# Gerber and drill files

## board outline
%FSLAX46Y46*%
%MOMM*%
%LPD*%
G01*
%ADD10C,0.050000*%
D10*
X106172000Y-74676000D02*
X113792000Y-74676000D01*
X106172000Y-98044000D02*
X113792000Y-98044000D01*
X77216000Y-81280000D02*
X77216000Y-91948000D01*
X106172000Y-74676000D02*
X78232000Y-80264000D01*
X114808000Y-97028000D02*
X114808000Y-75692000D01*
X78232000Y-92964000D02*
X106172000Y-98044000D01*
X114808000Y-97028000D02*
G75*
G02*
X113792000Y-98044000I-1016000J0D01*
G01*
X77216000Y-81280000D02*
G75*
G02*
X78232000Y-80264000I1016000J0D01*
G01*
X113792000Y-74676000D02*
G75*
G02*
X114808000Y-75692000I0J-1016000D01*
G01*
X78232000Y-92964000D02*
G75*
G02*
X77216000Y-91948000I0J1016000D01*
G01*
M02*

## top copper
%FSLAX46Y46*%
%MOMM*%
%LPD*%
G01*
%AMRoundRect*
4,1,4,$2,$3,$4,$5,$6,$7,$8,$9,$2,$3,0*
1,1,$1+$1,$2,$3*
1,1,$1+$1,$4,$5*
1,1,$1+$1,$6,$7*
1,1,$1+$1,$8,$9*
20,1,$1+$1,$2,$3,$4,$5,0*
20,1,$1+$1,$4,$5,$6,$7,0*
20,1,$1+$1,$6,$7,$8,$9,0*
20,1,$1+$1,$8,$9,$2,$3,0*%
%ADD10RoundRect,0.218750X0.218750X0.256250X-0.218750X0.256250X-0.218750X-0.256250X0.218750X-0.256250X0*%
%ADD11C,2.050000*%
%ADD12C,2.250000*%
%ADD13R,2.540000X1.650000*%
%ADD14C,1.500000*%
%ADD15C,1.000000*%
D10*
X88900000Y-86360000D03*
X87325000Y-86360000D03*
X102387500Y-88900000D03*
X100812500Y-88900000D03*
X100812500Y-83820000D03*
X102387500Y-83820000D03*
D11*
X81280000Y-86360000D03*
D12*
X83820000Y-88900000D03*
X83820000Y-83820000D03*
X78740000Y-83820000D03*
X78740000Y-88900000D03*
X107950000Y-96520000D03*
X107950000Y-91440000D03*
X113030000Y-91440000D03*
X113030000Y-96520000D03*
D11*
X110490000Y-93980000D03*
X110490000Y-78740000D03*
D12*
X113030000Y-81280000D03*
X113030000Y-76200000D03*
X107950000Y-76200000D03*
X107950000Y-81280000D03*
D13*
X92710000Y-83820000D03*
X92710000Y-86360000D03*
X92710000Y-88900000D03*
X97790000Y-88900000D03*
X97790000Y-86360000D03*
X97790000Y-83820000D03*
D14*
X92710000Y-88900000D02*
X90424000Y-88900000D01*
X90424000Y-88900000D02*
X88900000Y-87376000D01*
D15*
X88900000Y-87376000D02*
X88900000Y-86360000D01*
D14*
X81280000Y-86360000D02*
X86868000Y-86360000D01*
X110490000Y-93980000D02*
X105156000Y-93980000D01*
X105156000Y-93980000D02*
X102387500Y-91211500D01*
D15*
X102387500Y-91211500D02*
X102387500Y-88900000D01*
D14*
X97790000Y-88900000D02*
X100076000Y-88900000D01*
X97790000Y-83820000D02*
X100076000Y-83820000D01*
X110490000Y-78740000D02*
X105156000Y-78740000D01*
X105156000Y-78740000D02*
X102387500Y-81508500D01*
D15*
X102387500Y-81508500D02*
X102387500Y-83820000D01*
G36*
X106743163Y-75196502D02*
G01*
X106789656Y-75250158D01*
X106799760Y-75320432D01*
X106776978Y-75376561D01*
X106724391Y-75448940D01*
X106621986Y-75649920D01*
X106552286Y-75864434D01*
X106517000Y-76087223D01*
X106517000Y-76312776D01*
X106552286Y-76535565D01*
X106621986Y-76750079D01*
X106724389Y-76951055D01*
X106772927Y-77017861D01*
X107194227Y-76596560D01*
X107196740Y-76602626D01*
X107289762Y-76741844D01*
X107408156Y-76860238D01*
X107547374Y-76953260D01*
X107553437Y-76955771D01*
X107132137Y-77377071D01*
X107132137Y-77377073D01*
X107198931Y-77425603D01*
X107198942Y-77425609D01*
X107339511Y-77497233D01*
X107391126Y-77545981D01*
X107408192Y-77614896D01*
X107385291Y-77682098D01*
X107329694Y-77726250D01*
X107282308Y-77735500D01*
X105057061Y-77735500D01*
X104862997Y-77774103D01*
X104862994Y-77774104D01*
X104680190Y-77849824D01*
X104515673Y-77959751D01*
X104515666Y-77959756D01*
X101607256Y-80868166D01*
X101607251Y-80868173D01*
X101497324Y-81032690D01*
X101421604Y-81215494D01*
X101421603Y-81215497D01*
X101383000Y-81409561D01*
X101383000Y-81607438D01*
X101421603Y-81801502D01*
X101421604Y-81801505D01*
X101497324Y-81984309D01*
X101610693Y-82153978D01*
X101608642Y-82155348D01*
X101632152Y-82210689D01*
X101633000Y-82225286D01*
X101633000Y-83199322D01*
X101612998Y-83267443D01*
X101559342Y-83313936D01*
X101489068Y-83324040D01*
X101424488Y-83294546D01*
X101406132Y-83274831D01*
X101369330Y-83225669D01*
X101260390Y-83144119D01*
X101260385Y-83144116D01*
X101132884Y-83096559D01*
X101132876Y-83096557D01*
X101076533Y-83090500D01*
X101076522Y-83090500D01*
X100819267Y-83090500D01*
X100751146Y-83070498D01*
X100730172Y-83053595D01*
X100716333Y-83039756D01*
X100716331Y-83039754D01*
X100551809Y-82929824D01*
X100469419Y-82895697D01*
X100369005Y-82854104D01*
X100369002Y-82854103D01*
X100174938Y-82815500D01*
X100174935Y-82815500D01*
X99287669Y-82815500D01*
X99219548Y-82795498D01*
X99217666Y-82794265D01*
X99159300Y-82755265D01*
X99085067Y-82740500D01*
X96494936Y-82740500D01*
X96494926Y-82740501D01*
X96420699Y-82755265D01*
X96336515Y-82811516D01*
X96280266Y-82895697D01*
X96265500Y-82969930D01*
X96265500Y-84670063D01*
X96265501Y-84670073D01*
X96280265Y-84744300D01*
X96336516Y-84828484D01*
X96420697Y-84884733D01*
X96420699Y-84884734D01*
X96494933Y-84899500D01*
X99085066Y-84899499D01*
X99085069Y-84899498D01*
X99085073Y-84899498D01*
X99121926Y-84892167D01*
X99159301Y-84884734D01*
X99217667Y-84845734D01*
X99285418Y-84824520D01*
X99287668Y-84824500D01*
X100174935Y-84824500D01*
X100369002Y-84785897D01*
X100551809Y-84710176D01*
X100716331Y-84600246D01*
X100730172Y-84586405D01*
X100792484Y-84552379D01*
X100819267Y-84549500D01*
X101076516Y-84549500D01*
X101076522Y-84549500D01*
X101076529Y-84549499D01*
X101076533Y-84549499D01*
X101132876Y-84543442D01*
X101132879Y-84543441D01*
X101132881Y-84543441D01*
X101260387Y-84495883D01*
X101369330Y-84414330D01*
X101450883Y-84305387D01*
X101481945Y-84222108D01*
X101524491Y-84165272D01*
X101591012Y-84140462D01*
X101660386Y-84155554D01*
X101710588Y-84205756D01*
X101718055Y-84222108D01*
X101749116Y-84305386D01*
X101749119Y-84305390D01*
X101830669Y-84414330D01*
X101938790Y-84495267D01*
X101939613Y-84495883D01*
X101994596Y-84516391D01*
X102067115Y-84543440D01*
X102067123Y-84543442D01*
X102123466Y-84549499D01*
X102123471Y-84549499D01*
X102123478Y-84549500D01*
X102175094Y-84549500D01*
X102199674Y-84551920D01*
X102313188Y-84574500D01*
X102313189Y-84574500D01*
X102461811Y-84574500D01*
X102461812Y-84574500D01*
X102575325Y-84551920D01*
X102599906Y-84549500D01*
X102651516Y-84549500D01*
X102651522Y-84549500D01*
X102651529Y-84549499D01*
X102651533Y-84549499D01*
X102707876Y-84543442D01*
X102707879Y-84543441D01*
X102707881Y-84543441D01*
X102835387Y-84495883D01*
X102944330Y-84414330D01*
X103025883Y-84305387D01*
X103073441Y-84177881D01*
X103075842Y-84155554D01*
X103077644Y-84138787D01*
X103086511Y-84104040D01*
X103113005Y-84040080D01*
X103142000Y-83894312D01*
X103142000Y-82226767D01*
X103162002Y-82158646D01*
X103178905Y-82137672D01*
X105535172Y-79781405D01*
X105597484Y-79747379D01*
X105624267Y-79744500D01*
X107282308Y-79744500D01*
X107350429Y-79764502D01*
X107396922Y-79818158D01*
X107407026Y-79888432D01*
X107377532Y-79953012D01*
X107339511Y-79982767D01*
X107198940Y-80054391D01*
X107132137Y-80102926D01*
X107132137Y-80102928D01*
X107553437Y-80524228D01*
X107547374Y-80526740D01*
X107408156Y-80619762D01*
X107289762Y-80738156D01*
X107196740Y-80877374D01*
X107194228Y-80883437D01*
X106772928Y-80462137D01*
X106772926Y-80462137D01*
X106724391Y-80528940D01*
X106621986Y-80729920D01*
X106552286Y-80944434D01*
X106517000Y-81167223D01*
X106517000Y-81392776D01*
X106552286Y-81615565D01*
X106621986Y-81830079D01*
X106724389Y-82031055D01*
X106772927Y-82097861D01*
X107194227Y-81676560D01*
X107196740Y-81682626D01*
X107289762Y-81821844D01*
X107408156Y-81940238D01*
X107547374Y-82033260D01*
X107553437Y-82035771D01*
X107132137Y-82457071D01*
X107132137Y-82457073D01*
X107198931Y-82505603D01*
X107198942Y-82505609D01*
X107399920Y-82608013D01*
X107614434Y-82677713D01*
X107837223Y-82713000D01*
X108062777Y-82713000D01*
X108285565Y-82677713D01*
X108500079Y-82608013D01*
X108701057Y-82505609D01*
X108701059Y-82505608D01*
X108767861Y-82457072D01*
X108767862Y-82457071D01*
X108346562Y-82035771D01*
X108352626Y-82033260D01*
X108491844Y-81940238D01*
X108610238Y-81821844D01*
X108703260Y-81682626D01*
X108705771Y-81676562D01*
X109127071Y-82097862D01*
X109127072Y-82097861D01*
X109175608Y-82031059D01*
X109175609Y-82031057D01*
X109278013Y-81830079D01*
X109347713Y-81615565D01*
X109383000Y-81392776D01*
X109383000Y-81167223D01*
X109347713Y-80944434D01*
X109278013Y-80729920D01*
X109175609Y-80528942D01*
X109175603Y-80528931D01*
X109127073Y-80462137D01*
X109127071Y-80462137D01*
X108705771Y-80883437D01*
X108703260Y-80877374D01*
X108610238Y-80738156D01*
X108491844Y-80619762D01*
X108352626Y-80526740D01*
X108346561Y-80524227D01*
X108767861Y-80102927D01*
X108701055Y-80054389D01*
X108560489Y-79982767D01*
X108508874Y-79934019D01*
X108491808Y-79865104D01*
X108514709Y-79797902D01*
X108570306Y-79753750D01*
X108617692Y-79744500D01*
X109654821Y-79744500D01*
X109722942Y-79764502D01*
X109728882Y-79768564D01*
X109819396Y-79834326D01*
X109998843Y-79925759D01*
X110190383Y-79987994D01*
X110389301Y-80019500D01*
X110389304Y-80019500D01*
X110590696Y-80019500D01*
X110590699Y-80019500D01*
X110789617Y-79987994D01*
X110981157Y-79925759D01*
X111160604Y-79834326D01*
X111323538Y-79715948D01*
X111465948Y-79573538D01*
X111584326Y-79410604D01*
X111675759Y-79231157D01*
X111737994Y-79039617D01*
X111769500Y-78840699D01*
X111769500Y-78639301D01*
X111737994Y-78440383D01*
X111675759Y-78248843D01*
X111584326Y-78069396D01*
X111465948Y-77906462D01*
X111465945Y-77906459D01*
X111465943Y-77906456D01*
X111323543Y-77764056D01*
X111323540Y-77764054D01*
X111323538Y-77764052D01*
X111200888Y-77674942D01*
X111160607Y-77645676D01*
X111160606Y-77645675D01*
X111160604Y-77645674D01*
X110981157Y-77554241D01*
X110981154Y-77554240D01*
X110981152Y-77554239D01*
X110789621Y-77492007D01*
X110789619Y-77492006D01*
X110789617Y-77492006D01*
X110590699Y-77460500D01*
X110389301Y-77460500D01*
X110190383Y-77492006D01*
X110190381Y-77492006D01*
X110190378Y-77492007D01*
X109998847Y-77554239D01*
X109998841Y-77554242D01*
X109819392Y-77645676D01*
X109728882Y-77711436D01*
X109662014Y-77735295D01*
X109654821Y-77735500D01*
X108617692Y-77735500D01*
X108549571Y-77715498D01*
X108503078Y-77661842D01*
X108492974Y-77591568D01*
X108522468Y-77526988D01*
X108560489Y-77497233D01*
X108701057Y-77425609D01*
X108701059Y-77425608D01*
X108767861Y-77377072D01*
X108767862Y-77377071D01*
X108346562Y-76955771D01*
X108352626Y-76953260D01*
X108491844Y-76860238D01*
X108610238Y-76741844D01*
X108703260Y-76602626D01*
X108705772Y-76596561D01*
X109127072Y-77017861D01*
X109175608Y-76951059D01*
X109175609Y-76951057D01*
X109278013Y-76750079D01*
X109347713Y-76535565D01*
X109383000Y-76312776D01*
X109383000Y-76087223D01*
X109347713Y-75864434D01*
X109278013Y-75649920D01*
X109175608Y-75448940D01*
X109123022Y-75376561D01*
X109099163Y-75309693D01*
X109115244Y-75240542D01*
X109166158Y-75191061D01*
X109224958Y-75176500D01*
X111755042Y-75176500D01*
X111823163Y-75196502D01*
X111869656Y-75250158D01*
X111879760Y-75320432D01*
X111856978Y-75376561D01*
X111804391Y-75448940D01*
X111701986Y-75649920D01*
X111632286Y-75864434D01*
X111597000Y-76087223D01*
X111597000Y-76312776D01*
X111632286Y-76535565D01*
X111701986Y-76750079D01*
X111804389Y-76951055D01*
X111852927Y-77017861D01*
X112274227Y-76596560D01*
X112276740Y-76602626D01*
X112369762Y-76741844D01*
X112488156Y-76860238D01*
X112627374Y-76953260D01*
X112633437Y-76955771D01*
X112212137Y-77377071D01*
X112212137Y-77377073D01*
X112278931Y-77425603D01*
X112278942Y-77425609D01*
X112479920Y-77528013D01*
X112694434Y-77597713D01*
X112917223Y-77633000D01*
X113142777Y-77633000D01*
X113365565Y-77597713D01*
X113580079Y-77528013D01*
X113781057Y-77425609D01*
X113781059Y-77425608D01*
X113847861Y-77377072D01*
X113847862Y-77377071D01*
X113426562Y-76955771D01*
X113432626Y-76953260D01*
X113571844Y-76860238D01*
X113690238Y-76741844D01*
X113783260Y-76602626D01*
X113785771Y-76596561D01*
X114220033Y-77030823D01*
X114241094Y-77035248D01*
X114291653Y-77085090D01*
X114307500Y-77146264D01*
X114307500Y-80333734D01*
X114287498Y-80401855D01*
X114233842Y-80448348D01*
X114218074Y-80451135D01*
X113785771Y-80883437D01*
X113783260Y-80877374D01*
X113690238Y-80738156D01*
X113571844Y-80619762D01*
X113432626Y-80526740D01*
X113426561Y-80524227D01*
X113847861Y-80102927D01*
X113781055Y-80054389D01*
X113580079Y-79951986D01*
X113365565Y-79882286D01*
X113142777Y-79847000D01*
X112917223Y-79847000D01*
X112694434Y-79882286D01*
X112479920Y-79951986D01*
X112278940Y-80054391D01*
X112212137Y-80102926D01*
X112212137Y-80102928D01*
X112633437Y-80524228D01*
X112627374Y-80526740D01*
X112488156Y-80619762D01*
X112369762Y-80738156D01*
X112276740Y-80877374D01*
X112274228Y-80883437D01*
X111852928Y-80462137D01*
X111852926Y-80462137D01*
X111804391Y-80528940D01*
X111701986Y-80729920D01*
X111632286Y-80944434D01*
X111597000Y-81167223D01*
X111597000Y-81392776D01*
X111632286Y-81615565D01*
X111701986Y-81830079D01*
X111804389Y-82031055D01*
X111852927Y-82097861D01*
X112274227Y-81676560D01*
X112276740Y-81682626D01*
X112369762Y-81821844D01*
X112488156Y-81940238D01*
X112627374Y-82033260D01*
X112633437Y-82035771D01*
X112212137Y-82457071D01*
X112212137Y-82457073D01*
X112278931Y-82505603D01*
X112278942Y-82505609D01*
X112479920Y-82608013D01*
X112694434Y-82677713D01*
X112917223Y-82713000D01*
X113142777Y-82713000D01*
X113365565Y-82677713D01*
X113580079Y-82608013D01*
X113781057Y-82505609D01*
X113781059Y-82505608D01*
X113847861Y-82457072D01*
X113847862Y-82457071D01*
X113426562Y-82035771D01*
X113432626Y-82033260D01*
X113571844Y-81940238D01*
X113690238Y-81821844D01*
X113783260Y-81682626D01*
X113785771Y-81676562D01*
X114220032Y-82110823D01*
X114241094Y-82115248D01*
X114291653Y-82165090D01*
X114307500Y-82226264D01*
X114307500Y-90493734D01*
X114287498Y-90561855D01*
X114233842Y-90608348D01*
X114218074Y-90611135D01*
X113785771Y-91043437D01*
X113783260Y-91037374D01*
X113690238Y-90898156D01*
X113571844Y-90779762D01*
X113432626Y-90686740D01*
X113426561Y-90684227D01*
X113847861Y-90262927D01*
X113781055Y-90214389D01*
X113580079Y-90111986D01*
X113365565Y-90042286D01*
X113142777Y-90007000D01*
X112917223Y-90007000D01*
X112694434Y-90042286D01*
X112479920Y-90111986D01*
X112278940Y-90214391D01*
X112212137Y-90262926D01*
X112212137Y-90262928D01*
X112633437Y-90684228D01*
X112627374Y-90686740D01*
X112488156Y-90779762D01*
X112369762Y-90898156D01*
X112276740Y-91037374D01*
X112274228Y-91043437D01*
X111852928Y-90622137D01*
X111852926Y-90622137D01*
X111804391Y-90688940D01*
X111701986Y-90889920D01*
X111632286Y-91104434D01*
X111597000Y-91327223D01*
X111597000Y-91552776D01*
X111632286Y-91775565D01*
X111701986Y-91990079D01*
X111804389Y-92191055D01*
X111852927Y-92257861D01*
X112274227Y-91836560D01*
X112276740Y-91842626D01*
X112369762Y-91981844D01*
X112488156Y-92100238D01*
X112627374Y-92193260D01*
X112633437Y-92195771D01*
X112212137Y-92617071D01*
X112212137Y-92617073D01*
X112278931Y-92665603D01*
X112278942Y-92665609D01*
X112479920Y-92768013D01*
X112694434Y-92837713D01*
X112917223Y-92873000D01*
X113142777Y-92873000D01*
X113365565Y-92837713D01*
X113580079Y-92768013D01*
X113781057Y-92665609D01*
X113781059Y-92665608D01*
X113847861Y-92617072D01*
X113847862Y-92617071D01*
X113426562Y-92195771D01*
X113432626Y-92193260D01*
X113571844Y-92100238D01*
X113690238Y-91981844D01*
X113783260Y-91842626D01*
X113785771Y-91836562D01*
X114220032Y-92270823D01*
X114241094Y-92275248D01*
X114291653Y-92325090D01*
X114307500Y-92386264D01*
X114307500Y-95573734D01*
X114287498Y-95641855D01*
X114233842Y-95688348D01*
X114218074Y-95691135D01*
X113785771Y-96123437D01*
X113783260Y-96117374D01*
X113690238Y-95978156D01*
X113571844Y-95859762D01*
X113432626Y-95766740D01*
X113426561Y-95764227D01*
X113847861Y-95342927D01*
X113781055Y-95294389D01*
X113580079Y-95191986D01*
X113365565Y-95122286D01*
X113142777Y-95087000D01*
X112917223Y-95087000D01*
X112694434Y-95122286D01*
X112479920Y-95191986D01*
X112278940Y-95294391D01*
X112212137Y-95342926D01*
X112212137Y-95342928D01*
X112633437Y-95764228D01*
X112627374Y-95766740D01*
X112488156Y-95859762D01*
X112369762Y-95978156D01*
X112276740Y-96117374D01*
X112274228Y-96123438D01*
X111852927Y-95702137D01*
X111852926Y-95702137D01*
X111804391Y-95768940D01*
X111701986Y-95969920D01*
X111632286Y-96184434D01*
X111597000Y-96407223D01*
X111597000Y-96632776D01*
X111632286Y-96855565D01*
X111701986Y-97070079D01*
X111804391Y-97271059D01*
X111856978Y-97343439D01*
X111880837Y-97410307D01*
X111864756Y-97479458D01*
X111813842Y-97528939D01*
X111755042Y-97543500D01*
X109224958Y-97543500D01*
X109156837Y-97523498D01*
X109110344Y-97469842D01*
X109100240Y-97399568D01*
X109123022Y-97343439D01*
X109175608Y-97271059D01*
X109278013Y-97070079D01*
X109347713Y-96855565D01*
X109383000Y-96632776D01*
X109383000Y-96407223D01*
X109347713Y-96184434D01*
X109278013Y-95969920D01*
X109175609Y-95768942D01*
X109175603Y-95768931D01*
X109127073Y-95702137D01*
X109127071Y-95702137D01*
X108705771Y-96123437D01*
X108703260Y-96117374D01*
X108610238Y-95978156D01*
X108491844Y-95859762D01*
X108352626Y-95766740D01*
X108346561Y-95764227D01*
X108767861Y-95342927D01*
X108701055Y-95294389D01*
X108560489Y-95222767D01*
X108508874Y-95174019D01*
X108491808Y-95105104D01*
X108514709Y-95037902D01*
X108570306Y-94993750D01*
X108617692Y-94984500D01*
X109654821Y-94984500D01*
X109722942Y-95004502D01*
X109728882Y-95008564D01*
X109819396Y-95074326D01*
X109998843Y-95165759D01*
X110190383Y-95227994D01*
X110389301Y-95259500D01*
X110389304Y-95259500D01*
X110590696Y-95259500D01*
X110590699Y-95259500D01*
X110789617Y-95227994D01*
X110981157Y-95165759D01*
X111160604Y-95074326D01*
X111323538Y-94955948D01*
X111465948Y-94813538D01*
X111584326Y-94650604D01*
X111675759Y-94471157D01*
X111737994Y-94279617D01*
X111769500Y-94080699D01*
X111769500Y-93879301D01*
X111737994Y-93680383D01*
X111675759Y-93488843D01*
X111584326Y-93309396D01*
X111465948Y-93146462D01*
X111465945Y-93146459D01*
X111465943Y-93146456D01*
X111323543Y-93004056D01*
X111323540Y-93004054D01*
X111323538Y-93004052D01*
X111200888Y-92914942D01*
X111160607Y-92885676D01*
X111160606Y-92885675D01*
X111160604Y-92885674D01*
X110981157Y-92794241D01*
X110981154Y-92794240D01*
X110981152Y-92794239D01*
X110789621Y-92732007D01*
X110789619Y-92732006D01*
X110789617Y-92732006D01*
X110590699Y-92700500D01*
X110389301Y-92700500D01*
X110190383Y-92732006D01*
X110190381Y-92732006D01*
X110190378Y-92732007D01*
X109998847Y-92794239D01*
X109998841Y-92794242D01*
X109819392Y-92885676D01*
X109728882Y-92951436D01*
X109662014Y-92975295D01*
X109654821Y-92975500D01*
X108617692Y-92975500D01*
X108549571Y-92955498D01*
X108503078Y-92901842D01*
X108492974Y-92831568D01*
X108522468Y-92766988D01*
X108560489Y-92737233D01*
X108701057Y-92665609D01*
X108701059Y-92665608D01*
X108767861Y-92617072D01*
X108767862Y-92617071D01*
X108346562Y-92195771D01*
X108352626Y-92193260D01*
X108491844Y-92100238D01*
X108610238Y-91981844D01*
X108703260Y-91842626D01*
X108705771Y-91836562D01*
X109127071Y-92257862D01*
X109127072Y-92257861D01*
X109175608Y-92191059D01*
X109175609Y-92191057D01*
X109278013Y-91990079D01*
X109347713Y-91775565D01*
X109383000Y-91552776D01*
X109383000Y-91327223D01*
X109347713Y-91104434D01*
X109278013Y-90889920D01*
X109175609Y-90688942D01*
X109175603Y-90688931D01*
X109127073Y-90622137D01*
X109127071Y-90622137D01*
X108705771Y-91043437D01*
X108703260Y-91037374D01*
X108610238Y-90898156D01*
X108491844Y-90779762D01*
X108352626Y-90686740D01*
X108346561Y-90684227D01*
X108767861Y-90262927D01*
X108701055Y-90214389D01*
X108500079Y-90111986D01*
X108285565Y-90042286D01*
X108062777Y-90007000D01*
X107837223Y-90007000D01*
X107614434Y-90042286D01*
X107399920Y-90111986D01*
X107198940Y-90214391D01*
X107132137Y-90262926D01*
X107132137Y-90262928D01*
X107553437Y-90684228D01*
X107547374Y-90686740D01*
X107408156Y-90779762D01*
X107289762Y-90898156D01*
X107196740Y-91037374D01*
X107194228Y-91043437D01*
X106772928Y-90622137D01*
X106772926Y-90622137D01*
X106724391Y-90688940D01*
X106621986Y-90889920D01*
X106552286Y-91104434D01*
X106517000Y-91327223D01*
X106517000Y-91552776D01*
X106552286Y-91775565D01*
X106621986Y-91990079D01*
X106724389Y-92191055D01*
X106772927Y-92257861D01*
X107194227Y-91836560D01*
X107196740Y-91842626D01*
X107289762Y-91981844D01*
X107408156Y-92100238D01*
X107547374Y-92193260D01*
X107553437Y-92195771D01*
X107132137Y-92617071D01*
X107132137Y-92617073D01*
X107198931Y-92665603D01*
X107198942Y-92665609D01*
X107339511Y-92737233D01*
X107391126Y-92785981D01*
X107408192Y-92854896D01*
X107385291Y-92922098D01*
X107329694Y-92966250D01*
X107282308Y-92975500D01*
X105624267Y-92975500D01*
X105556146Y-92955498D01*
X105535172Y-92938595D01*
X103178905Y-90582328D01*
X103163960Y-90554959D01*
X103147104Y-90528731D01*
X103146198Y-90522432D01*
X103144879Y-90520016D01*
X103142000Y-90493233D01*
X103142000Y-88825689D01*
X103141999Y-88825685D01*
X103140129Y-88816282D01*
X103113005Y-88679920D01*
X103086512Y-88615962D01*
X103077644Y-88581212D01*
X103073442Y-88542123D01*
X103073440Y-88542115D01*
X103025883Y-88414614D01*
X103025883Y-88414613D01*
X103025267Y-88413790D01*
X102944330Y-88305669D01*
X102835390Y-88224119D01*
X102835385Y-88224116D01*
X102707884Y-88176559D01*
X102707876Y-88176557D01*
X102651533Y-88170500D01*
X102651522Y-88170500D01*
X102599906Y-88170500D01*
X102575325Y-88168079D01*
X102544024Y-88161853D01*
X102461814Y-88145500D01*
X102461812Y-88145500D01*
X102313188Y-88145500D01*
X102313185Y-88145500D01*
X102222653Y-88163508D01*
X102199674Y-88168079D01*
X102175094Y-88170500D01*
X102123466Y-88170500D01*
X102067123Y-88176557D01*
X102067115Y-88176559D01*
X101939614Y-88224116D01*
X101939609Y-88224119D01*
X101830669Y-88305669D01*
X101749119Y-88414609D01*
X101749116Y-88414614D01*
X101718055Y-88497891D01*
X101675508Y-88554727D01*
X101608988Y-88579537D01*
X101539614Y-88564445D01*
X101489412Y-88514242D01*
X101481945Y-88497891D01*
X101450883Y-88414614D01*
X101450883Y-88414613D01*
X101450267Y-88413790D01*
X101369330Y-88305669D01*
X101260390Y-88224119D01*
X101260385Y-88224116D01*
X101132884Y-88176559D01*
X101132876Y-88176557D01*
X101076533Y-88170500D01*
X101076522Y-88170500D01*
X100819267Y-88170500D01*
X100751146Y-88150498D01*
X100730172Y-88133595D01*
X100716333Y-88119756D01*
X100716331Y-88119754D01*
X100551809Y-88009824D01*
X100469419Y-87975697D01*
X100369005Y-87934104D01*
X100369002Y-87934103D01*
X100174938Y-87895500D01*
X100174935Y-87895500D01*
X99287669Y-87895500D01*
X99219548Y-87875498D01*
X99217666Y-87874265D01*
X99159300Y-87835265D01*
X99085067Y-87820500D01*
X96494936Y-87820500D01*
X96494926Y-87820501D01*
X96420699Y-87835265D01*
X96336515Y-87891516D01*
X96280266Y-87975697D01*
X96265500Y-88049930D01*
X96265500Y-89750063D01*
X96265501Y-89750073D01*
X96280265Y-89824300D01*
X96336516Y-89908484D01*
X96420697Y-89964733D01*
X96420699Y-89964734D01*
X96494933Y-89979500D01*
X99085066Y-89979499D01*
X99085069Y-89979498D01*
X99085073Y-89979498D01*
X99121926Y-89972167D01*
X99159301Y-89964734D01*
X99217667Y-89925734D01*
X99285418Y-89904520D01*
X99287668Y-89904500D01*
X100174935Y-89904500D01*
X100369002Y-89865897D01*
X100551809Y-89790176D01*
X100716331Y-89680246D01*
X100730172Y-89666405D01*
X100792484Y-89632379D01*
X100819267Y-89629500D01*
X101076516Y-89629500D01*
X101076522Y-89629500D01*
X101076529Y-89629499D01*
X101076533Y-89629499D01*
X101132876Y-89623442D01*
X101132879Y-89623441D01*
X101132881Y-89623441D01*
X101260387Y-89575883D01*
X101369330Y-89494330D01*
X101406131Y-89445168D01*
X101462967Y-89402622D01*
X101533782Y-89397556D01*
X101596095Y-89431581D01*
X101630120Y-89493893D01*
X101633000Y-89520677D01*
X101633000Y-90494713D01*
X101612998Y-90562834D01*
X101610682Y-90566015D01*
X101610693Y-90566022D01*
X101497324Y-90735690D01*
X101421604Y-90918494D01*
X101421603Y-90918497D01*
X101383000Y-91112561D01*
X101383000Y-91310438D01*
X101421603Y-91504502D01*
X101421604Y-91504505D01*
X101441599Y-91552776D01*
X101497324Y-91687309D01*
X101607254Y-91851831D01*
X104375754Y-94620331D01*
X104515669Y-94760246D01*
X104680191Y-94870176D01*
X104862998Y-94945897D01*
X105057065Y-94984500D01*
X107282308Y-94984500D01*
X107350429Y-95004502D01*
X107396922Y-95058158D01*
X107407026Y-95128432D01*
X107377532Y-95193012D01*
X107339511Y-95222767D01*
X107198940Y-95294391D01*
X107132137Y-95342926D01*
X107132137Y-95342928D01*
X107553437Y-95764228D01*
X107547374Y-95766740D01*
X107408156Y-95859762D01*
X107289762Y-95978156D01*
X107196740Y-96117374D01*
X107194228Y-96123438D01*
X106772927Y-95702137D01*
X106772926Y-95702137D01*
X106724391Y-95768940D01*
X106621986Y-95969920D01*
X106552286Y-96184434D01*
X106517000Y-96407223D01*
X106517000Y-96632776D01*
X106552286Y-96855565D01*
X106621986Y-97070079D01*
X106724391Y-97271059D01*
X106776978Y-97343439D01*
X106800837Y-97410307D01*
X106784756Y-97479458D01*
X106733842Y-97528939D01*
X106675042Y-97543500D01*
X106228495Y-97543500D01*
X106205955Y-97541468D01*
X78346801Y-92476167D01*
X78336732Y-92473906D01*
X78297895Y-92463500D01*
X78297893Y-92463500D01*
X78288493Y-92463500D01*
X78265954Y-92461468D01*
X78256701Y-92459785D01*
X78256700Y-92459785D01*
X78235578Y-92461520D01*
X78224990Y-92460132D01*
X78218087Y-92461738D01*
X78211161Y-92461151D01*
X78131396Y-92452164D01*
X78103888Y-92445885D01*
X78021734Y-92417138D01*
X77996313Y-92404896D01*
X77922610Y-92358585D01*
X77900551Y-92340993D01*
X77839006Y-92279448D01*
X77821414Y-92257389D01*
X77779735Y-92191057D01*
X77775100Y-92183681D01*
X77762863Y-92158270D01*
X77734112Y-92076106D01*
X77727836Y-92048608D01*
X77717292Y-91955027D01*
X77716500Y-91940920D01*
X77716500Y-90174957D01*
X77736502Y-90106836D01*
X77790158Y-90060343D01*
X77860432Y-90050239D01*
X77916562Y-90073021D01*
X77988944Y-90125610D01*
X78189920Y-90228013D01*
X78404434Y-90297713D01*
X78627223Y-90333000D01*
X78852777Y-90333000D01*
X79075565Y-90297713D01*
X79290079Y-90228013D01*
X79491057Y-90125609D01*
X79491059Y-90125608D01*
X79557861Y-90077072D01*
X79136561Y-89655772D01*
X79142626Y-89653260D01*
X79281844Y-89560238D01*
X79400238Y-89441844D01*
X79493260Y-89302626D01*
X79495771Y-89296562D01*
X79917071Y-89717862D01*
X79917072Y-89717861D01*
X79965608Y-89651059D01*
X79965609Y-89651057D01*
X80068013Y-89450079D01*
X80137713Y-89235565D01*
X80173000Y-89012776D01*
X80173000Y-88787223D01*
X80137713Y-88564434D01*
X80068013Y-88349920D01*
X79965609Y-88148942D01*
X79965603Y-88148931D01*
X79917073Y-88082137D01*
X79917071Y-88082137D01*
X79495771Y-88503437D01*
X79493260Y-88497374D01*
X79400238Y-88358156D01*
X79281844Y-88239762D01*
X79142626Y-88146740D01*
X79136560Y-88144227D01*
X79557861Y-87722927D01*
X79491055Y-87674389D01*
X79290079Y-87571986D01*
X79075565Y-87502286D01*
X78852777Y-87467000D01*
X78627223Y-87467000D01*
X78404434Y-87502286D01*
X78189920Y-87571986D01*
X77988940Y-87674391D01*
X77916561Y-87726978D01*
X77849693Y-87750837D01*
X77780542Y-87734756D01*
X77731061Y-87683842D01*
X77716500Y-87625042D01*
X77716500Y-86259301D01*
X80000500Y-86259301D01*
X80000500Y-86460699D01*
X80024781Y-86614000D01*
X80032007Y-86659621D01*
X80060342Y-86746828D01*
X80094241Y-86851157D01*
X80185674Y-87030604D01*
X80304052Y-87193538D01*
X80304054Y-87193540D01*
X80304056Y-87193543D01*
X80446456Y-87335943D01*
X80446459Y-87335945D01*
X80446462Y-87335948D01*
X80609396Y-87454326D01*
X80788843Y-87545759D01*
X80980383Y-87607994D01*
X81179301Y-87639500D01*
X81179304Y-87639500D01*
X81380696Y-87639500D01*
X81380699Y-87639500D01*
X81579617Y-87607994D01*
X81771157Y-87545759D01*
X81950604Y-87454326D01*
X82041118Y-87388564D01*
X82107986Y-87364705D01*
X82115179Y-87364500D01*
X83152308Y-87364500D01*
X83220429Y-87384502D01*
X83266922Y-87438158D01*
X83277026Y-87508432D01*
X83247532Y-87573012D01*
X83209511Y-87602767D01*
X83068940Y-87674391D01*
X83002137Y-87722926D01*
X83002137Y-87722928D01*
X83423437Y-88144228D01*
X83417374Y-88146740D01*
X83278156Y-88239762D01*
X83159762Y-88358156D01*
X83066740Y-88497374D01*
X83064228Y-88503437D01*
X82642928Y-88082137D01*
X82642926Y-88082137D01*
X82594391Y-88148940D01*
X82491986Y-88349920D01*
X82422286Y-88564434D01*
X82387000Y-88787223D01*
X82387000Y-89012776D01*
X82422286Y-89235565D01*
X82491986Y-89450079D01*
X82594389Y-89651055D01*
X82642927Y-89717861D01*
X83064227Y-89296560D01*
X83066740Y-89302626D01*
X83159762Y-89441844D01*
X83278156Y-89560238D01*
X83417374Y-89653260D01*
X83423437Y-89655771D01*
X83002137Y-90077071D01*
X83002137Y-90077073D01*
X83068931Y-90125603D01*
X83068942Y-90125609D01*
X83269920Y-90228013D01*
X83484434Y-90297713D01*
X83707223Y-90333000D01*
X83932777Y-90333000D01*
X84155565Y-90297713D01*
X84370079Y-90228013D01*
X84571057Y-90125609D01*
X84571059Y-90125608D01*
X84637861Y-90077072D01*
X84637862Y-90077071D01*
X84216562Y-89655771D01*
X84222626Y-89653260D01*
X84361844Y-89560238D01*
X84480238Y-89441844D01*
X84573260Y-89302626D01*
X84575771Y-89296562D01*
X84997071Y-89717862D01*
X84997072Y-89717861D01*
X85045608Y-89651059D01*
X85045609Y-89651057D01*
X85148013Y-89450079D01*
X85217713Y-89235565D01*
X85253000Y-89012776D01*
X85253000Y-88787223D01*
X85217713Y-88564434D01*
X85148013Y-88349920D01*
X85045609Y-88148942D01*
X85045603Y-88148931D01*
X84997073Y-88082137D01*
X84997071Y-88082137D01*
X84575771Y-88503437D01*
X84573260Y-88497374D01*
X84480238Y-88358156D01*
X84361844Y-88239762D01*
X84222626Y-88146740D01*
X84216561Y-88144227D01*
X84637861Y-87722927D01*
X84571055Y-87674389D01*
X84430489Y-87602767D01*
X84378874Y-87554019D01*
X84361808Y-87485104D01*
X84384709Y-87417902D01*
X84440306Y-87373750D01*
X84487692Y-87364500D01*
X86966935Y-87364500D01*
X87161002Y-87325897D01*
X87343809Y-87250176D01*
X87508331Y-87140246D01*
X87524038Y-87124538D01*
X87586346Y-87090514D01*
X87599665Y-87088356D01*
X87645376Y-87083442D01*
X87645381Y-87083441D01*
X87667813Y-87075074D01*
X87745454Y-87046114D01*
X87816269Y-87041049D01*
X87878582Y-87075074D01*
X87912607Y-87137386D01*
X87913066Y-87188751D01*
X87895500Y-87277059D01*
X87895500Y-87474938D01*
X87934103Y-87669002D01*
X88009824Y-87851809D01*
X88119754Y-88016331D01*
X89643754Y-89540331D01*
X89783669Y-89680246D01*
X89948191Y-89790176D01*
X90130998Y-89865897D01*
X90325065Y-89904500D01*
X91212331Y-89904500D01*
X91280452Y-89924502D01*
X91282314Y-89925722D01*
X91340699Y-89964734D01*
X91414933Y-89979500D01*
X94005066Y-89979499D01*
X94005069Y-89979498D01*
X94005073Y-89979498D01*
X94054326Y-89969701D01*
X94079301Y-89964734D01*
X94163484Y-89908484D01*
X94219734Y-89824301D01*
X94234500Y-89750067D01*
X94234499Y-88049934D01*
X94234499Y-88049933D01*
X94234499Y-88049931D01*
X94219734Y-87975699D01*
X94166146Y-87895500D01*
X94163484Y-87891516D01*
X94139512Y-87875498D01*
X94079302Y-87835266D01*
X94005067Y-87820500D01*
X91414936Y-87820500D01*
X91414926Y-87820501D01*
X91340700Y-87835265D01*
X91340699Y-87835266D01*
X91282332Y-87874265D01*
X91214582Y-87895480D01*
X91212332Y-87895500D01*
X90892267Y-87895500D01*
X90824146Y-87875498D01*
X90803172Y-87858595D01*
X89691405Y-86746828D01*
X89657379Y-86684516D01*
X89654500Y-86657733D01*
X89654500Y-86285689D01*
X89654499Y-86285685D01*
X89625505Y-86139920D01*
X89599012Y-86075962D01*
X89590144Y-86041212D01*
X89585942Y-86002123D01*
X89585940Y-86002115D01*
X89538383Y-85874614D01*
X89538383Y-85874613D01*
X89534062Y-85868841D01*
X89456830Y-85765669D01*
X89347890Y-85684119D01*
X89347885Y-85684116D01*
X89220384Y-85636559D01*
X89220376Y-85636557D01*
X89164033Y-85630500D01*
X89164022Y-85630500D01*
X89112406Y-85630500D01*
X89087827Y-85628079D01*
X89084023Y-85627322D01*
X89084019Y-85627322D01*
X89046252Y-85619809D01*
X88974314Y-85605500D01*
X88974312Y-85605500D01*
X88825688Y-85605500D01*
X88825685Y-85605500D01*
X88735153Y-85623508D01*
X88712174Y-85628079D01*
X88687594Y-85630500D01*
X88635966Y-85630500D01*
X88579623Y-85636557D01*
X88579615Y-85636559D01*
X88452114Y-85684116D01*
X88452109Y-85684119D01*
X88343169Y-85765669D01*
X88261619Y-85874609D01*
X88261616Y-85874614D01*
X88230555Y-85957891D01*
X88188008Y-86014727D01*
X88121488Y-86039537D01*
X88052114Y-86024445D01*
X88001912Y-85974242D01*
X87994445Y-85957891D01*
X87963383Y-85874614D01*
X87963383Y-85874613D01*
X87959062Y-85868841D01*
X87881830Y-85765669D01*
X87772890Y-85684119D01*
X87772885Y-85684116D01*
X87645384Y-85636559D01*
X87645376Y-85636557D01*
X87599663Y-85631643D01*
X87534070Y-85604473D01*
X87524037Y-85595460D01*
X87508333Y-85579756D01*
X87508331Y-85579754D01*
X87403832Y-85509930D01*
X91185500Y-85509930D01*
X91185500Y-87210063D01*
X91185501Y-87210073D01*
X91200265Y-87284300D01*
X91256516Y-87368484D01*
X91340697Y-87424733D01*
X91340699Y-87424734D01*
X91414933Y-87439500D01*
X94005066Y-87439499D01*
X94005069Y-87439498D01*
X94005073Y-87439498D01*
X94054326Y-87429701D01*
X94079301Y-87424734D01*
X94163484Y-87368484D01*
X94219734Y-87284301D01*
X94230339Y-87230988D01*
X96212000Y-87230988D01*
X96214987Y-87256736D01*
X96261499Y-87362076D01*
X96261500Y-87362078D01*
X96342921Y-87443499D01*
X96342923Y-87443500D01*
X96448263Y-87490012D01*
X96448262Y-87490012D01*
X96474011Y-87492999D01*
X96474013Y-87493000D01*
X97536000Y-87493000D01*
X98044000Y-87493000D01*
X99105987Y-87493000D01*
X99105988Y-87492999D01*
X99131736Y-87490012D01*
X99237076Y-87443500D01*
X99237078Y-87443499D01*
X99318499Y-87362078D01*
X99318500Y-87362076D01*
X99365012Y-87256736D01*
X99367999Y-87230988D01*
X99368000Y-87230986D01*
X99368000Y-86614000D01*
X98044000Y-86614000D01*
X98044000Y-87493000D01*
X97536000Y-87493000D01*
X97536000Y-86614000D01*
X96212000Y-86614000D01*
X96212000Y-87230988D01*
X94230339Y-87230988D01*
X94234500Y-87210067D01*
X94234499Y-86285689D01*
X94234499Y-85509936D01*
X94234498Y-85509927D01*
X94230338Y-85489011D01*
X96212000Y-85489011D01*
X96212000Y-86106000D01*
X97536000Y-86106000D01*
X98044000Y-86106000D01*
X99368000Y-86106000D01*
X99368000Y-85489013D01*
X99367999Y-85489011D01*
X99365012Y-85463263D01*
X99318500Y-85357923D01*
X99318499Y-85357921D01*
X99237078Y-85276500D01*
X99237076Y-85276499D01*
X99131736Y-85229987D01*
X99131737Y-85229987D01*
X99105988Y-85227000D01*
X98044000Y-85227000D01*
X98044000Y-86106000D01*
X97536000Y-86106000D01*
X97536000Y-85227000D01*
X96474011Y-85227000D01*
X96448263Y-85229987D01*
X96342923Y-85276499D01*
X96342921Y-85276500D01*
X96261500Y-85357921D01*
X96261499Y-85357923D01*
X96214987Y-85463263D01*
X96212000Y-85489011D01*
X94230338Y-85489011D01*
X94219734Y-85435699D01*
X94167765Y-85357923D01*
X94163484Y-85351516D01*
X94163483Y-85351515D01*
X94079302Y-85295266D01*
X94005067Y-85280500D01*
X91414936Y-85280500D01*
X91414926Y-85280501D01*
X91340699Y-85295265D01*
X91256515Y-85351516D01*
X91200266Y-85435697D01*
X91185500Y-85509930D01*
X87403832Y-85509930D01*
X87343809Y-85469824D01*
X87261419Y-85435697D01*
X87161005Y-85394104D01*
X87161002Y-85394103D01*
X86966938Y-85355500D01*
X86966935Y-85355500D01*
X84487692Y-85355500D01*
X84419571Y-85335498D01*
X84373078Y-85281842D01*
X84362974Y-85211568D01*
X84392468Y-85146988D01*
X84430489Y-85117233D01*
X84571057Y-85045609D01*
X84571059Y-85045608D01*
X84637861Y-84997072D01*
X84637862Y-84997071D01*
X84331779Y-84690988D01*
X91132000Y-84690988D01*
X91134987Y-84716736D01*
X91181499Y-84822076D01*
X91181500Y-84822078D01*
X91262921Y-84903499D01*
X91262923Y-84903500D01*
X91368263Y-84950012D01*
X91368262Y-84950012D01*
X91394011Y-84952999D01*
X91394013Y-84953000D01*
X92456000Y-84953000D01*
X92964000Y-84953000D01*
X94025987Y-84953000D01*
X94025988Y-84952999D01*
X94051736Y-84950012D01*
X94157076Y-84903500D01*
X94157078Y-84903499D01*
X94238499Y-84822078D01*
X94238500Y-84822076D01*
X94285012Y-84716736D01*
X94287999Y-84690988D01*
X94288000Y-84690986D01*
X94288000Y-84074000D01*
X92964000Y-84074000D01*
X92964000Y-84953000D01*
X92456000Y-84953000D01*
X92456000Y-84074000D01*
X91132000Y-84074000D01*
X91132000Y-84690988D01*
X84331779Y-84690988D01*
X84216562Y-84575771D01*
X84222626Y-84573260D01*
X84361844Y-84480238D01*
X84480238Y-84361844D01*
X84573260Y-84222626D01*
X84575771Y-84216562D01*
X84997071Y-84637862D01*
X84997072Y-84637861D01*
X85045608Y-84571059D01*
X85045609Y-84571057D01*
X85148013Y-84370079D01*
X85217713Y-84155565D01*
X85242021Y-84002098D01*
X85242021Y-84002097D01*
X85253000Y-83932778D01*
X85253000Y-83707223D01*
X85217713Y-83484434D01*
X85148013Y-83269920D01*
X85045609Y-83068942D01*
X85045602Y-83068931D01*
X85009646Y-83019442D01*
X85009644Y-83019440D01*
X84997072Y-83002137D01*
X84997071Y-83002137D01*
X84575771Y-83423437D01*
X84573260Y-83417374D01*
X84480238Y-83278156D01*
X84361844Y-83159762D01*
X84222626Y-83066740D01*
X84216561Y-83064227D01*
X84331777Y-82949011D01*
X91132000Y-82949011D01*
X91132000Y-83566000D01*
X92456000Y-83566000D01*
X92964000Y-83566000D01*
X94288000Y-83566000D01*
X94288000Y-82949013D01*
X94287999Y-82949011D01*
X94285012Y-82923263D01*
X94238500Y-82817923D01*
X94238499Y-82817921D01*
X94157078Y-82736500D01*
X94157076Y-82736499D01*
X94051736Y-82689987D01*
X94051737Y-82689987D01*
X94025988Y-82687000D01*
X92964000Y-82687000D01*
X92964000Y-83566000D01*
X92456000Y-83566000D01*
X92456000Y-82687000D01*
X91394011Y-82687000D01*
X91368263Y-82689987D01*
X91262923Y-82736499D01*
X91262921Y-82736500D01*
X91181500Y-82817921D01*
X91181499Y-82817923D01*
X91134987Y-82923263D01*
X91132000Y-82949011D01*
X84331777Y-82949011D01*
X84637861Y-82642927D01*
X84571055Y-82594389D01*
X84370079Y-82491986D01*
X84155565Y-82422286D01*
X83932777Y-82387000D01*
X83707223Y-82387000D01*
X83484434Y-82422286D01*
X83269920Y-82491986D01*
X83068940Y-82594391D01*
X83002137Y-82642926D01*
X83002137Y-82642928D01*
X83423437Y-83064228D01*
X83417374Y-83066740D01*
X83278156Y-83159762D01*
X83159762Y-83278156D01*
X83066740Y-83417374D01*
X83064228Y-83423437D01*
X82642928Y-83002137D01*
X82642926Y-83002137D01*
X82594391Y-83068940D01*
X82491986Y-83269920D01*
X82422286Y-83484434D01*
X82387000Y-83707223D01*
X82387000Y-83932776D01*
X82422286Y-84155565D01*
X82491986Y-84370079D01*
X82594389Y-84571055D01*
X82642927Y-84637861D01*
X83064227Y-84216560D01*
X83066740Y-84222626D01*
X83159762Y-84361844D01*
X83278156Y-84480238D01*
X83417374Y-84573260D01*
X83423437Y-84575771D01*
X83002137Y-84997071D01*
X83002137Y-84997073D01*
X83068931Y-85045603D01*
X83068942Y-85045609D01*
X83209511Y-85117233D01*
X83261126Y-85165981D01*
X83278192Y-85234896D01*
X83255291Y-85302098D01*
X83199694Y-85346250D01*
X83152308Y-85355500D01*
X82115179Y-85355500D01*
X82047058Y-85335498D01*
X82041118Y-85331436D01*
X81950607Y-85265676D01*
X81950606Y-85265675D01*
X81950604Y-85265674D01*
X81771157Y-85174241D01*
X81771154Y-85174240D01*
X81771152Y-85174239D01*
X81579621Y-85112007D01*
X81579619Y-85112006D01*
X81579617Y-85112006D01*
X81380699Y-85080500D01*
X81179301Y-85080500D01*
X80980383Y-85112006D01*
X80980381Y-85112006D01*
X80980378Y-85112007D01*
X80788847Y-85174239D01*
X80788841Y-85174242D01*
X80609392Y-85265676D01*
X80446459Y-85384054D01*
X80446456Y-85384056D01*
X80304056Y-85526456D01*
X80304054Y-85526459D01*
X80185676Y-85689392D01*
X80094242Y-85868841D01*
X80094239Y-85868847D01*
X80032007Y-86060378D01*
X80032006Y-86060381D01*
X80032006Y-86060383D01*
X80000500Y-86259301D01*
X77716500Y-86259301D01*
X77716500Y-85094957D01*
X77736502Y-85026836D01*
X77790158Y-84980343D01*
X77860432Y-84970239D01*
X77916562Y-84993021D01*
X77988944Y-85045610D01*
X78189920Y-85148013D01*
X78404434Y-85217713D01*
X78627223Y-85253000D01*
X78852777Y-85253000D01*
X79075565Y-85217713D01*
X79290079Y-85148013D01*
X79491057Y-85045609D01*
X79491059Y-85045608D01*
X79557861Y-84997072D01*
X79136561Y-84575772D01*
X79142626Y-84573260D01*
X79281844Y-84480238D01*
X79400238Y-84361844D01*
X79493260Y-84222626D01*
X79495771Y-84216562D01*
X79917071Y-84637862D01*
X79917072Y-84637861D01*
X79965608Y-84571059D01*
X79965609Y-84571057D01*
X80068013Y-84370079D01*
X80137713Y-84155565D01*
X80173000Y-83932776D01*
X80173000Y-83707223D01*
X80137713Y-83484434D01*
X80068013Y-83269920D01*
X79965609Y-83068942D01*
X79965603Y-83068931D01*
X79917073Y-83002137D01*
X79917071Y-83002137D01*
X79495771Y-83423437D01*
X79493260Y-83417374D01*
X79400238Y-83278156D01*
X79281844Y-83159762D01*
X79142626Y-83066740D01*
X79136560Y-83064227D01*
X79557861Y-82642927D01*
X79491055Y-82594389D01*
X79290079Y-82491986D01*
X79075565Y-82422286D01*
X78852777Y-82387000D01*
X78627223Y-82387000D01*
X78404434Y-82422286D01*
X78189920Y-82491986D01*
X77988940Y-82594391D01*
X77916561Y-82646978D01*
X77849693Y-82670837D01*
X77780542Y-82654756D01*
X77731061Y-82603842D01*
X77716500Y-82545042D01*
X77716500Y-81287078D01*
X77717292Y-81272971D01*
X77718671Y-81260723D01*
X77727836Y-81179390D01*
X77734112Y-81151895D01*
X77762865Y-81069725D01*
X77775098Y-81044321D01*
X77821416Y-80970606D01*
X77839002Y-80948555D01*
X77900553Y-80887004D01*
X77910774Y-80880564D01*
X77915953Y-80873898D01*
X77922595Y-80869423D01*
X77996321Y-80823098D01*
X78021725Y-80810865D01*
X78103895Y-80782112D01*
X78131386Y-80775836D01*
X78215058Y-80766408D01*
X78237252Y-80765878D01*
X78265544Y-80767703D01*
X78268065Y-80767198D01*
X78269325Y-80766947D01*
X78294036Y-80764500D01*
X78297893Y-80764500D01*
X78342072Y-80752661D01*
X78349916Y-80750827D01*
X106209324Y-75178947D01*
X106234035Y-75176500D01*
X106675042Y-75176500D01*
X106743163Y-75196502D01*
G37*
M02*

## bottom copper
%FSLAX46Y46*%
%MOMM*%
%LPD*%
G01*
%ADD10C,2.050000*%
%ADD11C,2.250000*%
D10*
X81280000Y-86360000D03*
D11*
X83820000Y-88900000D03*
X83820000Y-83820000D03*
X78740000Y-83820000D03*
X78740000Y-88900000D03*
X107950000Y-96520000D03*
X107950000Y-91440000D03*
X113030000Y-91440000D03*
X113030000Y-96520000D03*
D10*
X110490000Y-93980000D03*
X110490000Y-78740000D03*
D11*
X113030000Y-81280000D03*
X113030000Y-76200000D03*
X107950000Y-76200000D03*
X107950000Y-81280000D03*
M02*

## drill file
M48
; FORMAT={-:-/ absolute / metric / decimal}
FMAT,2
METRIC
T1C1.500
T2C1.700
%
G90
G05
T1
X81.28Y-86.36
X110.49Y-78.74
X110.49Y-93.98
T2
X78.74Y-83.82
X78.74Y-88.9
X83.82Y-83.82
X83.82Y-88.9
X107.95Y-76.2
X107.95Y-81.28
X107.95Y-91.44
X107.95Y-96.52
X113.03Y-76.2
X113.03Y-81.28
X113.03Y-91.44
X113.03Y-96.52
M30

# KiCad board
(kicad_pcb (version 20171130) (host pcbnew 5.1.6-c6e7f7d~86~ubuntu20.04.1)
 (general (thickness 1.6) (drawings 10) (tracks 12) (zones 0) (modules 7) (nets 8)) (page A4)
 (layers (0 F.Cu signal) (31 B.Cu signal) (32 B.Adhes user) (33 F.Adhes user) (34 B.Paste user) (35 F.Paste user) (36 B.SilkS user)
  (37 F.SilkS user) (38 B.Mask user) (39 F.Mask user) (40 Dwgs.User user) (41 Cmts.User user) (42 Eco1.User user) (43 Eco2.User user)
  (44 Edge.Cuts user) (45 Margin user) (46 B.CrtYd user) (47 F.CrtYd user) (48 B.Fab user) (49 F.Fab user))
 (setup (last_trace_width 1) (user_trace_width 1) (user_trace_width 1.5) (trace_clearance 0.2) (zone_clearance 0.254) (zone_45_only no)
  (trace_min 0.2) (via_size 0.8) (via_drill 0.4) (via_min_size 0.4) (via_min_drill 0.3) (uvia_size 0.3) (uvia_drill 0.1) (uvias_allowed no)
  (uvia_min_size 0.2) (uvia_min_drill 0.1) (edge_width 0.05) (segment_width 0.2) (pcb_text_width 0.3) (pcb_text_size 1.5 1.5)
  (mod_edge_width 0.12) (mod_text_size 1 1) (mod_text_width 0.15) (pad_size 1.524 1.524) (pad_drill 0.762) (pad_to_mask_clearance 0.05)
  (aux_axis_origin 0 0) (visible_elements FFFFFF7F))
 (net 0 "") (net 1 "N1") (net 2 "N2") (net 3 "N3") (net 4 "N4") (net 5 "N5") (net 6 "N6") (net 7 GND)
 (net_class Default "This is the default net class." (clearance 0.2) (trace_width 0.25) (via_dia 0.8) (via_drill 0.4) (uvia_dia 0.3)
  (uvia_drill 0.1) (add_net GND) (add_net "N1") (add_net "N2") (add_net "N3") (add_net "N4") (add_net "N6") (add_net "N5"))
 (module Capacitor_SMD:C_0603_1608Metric (layer F.Cu) (at 88.1125 86.36 180)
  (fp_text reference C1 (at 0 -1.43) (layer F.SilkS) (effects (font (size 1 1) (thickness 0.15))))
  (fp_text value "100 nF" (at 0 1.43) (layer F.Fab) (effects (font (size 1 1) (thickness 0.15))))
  (pad 1 smd roundrect (at -0.7875 0 180) (size 0.875 0.95) (layers F.Cu F.Paste F.Mask) (roundrect_rratio 0.25) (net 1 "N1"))
  (pad 2 smd roundrect (at 0.7875 0 180) (size 0.875 0.95) (layers F.Cu F.Paste F.Mask) (roundrect_rratio 0.25) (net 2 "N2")))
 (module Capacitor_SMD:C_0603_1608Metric (layer F.Cu) (at 101.6 88.9 180)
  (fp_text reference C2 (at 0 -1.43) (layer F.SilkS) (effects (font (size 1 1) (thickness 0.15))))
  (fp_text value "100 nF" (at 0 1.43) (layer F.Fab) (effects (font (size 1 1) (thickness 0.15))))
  (pad 1 smd roundrect (at -0.7875 0 180) (size 0.875 0.95) (layers F.Cu F.Paste F.Mask) (roundrect_rratio 0.25) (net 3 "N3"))
  (pad 2 smd roundrect (at 0.7875 0 180) (size 0.875 0.95) (layers F.Cu F.Paste F.Mask) (roundrect_rratio 0.25) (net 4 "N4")))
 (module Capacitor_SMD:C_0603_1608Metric (layer F.Cu) (at 101.6 83.82 180)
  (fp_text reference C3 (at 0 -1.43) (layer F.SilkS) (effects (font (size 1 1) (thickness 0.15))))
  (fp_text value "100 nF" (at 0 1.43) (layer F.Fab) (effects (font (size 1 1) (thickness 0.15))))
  (pad 2 smd roundrect (at 0.7875 0 180) (size 0.875 0.95) (layers F.Cu F.Paste F.Mask) (roundrect_rratio 0.25) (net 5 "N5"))
  (pad 1 smd roundrect (at -0.7875 0 180) (size 0.875 0.95) (layers F.Cu F.Paste F.Mask) (roundrect_rratio 0.25) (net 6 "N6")))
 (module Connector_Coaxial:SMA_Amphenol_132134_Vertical (layer F.Cu) (at 81.28 86.36)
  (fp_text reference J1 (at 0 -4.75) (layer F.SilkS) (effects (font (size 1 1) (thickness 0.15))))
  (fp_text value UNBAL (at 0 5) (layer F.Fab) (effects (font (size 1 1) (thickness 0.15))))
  (pad 1 thru_hole circle (at 0 0) (size 2.05 2.05) (drill 1.5) (layers *.Cu *.Mask) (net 2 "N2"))
  (pad 2 thru_hole circle (at 2.54 2.54) (size 2.25 2.25) (drill 1.7) (layers *.Cu *.Mask) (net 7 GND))
  (pad 2 thru_hole circle (at 2.54 -2.54) (size 2.25 2.25) (drill 1.7) (layers *.Cu *.Mask) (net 7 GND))
  (pad 2 thru_hole circle (at -2.54 -2.54) (size 2.25 2.25) (drill 1.7) (layers *.Cu *.Mask) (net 7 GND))
  (pad 2 thru_hole circle (at -2.54 2.54) (size 2.25 2.25) (drill 1.7) (layers *.Cu *.Mask) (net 7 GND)))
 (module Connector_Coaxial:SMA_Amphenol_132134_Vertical (layer F.Cu) (at 110.49 93.98)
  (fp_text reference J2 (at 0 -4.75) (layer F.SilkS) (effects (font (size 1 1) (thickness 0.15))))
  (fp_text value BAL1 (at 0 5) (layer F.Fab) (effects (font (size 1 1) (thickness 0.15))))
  (pad 2 thru_hole circle (at -2.54 2.54) (size 2.25 2.25) (drill 1.7) (layers *.Cu *.Mask) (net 7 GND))
  (pad 2 thru_hole circle (at -2.54 -2.54) (size 2.25 2.25) (drill 1.7) (layers *.Cu *.Mask) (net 7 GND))
  (pad 2 thru_hole circle (at 2.54 -2.54) (size 2.25 2.25) (drill 1.7) (layers *.Cu *.Mask) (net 7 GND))
  (pad 2 thru_hole circle (at 2.54 2.54) (size 2.25 2.25) (drill 1.7) (layers *.Cu *.Mask) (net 7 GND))
  (pad 1 thru_hole circle (at 0 0) (size 2.05 2.05) (drill 1.5) (layers *.Cu *.Mask) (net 3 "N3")))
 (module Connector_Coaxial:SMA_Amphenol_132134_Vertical (layer F.Cu) (at 110.49 78.74)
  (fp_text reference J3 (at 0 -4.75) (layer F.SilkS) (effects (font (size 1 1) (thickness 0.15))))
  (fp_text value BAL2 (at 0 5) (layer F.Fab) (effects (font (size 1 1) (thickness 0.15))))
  (pad 1 thru_hole circle (at 0 0) (size 2.05 2.05) (drill 1.5) (layers *.Cu *.Mask) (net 6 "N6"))
  (pad 2 thru_hole circle (at 2.54 2.54) (size 2.25 2.25) (drill 1.7) (layers *.Cu *.Mask) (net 7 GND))
  (pad 2 thru_hole circle (at 2.54 -2.54) (size 2.25 2.25) (drill 1.7) (layers *.Cu *.Mask) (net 7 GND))
  (pad 2 thru_hole circle (at -2.54 -2.54) (size 2.25 2.25) (drill 1.7) (layers *.Cu *.Mask) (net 7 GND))
  (pad 2 thru_hole circle (at -2.54 2.54) (size 2.25 2.25) (drill 1.7) (layers *.Cu *.Mask) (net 7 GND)))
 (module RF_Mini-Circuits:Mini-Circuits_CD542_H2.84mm (layer F.Cu) (at 95.25 86.36)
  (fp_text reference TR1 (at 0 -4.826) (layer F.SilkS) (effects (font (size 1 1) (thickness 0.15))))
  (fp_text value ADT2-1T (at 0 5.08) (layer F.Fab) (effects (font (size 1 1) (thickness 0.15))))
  (pad 1 smd rect (at -2.54 -2.54) (size 2.54 1.65) (layers F.Cu F.Paste F.Mask) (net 7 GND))
  (pad 2 smd rect (at -2.54 0) (size 2.54 1.65) (layers F.Cu F.Paste F.Mask))
  (pad 3 smd rect (at -2.54 2.54) (size 2.54 1.65) (layers F.Cu F.Paste F.Mask) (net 1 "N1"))
  (pad 4 smd rect (at 2.54 2.54) (size 2.54 1.65) (layers F.Cu F.Paste F.Mask) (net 4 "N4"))
  (pad 5 smd rect (at 2.54 0) (size 2.54 1.65) (layers F.Cu F.Paste F.Mask) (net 7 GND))
  (pad 6 smd rect (at 2.54 -2.54) (size 2.54 1.65) (layers F.Cu F.Paste F.Mask) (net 5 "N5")))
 (gr_line (start 106.172 74.676) (end 113.792 74.676) (layer Edge.Cuts) (width 0.05))
 (gr_line (start 106.172 98.044) (end 113.792 98.044) (layer Edge.Cuts) (width 0.05))
 (gr_line (start 77.216 81.28) (end 77.216 91.948) (layer Edge.Cuts) (width 0.05))
 (gr_line (start 106.172 74.676) (end 78.232 80.264) (layer Edge.Cuts) (width 0.05))
 (gr_line (start 114.808 97.028) (end 114.808 75.692) (layer Edge.Cuts) (width 0.05))
 (gr_line (start 78.232 92.964) (end 106.172 98.044) (layer Edge.Cuts) (width 0.05))
 (gr_arc (start 113.792 97.028) (end 113.792 98.044) (angle -90) (layer Edge.Cuts) (width 0.05))
 (gr_arc (start 78.232 81.28) (end 78.232 80.264) (angle -90) (layer Edge.Cuts) (width 0.05))
 (gr_arc (start 113.792 75.692) (end 114.808 75.692) (angle -90) (layer Edge.Cuts) (width 0.05))
 (gr_arc (start 78.232 91.948) (end 77.216 91.948) (angle -90) (layer Edge.Cuts) (width 0.05))
 (segment (start 92.71 88.9) (end 90.424 88.9) (width 1.5) (layer F.Cu) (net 1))
 (segment (start 90.424 88.9) (end 88.9 87.376) (width 1.5) (layer F.Cu) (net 1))
 (segment (start 88.9 87.376) (end 88.9 86.36) (width 1) (layer F.Cu) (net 1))
 (segment (start 81.28 86.36) (end 86.868 86.36) (width 1.5) (layer F.Cu) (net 2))
 (segment (start 110.49 93.98) (end 105.156 93.98) (width 1.5) (layer F.Cu) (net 3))
 (segment (start 105.156 93.98) (end 102.3875 91.2115) (width 1.5) (layer F.Cu) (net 3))
 (segment (start 102.3875 91.2115) (end 102.3875 88.9) (width 1) (layer F.Cu) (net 3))
 (segment (start 97.79 88.9) (end 100.076 88.9) (width 1.5) (layer F.Cu) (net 4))
 (segment (start 97.79 83.82) (end 100.076 83.82) (width 1.5) (layer F.Cu) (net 5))
 (segment (start 110.49 78.74) (end 105.156 78.74) (width 1.5) (layer F.Cu) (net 6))
 (segment (start 105.156 78.74) (end 102.3875 81.5085) (width 1.5) (layer F.Cu) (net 6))
 (segment (start 102.3875 81.5085) (end 102.3875 83.82) (width 1) (layer F.Cu) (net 6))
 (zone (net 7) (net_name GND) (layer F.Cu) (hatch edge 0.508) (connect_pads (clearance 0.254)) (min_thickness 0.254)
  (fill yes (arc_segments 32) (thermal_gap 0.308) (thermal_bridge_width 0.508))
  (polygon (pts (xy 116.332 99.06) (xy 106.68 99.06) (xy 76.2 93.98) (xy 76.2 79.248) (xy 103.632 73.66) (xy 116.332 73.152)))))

